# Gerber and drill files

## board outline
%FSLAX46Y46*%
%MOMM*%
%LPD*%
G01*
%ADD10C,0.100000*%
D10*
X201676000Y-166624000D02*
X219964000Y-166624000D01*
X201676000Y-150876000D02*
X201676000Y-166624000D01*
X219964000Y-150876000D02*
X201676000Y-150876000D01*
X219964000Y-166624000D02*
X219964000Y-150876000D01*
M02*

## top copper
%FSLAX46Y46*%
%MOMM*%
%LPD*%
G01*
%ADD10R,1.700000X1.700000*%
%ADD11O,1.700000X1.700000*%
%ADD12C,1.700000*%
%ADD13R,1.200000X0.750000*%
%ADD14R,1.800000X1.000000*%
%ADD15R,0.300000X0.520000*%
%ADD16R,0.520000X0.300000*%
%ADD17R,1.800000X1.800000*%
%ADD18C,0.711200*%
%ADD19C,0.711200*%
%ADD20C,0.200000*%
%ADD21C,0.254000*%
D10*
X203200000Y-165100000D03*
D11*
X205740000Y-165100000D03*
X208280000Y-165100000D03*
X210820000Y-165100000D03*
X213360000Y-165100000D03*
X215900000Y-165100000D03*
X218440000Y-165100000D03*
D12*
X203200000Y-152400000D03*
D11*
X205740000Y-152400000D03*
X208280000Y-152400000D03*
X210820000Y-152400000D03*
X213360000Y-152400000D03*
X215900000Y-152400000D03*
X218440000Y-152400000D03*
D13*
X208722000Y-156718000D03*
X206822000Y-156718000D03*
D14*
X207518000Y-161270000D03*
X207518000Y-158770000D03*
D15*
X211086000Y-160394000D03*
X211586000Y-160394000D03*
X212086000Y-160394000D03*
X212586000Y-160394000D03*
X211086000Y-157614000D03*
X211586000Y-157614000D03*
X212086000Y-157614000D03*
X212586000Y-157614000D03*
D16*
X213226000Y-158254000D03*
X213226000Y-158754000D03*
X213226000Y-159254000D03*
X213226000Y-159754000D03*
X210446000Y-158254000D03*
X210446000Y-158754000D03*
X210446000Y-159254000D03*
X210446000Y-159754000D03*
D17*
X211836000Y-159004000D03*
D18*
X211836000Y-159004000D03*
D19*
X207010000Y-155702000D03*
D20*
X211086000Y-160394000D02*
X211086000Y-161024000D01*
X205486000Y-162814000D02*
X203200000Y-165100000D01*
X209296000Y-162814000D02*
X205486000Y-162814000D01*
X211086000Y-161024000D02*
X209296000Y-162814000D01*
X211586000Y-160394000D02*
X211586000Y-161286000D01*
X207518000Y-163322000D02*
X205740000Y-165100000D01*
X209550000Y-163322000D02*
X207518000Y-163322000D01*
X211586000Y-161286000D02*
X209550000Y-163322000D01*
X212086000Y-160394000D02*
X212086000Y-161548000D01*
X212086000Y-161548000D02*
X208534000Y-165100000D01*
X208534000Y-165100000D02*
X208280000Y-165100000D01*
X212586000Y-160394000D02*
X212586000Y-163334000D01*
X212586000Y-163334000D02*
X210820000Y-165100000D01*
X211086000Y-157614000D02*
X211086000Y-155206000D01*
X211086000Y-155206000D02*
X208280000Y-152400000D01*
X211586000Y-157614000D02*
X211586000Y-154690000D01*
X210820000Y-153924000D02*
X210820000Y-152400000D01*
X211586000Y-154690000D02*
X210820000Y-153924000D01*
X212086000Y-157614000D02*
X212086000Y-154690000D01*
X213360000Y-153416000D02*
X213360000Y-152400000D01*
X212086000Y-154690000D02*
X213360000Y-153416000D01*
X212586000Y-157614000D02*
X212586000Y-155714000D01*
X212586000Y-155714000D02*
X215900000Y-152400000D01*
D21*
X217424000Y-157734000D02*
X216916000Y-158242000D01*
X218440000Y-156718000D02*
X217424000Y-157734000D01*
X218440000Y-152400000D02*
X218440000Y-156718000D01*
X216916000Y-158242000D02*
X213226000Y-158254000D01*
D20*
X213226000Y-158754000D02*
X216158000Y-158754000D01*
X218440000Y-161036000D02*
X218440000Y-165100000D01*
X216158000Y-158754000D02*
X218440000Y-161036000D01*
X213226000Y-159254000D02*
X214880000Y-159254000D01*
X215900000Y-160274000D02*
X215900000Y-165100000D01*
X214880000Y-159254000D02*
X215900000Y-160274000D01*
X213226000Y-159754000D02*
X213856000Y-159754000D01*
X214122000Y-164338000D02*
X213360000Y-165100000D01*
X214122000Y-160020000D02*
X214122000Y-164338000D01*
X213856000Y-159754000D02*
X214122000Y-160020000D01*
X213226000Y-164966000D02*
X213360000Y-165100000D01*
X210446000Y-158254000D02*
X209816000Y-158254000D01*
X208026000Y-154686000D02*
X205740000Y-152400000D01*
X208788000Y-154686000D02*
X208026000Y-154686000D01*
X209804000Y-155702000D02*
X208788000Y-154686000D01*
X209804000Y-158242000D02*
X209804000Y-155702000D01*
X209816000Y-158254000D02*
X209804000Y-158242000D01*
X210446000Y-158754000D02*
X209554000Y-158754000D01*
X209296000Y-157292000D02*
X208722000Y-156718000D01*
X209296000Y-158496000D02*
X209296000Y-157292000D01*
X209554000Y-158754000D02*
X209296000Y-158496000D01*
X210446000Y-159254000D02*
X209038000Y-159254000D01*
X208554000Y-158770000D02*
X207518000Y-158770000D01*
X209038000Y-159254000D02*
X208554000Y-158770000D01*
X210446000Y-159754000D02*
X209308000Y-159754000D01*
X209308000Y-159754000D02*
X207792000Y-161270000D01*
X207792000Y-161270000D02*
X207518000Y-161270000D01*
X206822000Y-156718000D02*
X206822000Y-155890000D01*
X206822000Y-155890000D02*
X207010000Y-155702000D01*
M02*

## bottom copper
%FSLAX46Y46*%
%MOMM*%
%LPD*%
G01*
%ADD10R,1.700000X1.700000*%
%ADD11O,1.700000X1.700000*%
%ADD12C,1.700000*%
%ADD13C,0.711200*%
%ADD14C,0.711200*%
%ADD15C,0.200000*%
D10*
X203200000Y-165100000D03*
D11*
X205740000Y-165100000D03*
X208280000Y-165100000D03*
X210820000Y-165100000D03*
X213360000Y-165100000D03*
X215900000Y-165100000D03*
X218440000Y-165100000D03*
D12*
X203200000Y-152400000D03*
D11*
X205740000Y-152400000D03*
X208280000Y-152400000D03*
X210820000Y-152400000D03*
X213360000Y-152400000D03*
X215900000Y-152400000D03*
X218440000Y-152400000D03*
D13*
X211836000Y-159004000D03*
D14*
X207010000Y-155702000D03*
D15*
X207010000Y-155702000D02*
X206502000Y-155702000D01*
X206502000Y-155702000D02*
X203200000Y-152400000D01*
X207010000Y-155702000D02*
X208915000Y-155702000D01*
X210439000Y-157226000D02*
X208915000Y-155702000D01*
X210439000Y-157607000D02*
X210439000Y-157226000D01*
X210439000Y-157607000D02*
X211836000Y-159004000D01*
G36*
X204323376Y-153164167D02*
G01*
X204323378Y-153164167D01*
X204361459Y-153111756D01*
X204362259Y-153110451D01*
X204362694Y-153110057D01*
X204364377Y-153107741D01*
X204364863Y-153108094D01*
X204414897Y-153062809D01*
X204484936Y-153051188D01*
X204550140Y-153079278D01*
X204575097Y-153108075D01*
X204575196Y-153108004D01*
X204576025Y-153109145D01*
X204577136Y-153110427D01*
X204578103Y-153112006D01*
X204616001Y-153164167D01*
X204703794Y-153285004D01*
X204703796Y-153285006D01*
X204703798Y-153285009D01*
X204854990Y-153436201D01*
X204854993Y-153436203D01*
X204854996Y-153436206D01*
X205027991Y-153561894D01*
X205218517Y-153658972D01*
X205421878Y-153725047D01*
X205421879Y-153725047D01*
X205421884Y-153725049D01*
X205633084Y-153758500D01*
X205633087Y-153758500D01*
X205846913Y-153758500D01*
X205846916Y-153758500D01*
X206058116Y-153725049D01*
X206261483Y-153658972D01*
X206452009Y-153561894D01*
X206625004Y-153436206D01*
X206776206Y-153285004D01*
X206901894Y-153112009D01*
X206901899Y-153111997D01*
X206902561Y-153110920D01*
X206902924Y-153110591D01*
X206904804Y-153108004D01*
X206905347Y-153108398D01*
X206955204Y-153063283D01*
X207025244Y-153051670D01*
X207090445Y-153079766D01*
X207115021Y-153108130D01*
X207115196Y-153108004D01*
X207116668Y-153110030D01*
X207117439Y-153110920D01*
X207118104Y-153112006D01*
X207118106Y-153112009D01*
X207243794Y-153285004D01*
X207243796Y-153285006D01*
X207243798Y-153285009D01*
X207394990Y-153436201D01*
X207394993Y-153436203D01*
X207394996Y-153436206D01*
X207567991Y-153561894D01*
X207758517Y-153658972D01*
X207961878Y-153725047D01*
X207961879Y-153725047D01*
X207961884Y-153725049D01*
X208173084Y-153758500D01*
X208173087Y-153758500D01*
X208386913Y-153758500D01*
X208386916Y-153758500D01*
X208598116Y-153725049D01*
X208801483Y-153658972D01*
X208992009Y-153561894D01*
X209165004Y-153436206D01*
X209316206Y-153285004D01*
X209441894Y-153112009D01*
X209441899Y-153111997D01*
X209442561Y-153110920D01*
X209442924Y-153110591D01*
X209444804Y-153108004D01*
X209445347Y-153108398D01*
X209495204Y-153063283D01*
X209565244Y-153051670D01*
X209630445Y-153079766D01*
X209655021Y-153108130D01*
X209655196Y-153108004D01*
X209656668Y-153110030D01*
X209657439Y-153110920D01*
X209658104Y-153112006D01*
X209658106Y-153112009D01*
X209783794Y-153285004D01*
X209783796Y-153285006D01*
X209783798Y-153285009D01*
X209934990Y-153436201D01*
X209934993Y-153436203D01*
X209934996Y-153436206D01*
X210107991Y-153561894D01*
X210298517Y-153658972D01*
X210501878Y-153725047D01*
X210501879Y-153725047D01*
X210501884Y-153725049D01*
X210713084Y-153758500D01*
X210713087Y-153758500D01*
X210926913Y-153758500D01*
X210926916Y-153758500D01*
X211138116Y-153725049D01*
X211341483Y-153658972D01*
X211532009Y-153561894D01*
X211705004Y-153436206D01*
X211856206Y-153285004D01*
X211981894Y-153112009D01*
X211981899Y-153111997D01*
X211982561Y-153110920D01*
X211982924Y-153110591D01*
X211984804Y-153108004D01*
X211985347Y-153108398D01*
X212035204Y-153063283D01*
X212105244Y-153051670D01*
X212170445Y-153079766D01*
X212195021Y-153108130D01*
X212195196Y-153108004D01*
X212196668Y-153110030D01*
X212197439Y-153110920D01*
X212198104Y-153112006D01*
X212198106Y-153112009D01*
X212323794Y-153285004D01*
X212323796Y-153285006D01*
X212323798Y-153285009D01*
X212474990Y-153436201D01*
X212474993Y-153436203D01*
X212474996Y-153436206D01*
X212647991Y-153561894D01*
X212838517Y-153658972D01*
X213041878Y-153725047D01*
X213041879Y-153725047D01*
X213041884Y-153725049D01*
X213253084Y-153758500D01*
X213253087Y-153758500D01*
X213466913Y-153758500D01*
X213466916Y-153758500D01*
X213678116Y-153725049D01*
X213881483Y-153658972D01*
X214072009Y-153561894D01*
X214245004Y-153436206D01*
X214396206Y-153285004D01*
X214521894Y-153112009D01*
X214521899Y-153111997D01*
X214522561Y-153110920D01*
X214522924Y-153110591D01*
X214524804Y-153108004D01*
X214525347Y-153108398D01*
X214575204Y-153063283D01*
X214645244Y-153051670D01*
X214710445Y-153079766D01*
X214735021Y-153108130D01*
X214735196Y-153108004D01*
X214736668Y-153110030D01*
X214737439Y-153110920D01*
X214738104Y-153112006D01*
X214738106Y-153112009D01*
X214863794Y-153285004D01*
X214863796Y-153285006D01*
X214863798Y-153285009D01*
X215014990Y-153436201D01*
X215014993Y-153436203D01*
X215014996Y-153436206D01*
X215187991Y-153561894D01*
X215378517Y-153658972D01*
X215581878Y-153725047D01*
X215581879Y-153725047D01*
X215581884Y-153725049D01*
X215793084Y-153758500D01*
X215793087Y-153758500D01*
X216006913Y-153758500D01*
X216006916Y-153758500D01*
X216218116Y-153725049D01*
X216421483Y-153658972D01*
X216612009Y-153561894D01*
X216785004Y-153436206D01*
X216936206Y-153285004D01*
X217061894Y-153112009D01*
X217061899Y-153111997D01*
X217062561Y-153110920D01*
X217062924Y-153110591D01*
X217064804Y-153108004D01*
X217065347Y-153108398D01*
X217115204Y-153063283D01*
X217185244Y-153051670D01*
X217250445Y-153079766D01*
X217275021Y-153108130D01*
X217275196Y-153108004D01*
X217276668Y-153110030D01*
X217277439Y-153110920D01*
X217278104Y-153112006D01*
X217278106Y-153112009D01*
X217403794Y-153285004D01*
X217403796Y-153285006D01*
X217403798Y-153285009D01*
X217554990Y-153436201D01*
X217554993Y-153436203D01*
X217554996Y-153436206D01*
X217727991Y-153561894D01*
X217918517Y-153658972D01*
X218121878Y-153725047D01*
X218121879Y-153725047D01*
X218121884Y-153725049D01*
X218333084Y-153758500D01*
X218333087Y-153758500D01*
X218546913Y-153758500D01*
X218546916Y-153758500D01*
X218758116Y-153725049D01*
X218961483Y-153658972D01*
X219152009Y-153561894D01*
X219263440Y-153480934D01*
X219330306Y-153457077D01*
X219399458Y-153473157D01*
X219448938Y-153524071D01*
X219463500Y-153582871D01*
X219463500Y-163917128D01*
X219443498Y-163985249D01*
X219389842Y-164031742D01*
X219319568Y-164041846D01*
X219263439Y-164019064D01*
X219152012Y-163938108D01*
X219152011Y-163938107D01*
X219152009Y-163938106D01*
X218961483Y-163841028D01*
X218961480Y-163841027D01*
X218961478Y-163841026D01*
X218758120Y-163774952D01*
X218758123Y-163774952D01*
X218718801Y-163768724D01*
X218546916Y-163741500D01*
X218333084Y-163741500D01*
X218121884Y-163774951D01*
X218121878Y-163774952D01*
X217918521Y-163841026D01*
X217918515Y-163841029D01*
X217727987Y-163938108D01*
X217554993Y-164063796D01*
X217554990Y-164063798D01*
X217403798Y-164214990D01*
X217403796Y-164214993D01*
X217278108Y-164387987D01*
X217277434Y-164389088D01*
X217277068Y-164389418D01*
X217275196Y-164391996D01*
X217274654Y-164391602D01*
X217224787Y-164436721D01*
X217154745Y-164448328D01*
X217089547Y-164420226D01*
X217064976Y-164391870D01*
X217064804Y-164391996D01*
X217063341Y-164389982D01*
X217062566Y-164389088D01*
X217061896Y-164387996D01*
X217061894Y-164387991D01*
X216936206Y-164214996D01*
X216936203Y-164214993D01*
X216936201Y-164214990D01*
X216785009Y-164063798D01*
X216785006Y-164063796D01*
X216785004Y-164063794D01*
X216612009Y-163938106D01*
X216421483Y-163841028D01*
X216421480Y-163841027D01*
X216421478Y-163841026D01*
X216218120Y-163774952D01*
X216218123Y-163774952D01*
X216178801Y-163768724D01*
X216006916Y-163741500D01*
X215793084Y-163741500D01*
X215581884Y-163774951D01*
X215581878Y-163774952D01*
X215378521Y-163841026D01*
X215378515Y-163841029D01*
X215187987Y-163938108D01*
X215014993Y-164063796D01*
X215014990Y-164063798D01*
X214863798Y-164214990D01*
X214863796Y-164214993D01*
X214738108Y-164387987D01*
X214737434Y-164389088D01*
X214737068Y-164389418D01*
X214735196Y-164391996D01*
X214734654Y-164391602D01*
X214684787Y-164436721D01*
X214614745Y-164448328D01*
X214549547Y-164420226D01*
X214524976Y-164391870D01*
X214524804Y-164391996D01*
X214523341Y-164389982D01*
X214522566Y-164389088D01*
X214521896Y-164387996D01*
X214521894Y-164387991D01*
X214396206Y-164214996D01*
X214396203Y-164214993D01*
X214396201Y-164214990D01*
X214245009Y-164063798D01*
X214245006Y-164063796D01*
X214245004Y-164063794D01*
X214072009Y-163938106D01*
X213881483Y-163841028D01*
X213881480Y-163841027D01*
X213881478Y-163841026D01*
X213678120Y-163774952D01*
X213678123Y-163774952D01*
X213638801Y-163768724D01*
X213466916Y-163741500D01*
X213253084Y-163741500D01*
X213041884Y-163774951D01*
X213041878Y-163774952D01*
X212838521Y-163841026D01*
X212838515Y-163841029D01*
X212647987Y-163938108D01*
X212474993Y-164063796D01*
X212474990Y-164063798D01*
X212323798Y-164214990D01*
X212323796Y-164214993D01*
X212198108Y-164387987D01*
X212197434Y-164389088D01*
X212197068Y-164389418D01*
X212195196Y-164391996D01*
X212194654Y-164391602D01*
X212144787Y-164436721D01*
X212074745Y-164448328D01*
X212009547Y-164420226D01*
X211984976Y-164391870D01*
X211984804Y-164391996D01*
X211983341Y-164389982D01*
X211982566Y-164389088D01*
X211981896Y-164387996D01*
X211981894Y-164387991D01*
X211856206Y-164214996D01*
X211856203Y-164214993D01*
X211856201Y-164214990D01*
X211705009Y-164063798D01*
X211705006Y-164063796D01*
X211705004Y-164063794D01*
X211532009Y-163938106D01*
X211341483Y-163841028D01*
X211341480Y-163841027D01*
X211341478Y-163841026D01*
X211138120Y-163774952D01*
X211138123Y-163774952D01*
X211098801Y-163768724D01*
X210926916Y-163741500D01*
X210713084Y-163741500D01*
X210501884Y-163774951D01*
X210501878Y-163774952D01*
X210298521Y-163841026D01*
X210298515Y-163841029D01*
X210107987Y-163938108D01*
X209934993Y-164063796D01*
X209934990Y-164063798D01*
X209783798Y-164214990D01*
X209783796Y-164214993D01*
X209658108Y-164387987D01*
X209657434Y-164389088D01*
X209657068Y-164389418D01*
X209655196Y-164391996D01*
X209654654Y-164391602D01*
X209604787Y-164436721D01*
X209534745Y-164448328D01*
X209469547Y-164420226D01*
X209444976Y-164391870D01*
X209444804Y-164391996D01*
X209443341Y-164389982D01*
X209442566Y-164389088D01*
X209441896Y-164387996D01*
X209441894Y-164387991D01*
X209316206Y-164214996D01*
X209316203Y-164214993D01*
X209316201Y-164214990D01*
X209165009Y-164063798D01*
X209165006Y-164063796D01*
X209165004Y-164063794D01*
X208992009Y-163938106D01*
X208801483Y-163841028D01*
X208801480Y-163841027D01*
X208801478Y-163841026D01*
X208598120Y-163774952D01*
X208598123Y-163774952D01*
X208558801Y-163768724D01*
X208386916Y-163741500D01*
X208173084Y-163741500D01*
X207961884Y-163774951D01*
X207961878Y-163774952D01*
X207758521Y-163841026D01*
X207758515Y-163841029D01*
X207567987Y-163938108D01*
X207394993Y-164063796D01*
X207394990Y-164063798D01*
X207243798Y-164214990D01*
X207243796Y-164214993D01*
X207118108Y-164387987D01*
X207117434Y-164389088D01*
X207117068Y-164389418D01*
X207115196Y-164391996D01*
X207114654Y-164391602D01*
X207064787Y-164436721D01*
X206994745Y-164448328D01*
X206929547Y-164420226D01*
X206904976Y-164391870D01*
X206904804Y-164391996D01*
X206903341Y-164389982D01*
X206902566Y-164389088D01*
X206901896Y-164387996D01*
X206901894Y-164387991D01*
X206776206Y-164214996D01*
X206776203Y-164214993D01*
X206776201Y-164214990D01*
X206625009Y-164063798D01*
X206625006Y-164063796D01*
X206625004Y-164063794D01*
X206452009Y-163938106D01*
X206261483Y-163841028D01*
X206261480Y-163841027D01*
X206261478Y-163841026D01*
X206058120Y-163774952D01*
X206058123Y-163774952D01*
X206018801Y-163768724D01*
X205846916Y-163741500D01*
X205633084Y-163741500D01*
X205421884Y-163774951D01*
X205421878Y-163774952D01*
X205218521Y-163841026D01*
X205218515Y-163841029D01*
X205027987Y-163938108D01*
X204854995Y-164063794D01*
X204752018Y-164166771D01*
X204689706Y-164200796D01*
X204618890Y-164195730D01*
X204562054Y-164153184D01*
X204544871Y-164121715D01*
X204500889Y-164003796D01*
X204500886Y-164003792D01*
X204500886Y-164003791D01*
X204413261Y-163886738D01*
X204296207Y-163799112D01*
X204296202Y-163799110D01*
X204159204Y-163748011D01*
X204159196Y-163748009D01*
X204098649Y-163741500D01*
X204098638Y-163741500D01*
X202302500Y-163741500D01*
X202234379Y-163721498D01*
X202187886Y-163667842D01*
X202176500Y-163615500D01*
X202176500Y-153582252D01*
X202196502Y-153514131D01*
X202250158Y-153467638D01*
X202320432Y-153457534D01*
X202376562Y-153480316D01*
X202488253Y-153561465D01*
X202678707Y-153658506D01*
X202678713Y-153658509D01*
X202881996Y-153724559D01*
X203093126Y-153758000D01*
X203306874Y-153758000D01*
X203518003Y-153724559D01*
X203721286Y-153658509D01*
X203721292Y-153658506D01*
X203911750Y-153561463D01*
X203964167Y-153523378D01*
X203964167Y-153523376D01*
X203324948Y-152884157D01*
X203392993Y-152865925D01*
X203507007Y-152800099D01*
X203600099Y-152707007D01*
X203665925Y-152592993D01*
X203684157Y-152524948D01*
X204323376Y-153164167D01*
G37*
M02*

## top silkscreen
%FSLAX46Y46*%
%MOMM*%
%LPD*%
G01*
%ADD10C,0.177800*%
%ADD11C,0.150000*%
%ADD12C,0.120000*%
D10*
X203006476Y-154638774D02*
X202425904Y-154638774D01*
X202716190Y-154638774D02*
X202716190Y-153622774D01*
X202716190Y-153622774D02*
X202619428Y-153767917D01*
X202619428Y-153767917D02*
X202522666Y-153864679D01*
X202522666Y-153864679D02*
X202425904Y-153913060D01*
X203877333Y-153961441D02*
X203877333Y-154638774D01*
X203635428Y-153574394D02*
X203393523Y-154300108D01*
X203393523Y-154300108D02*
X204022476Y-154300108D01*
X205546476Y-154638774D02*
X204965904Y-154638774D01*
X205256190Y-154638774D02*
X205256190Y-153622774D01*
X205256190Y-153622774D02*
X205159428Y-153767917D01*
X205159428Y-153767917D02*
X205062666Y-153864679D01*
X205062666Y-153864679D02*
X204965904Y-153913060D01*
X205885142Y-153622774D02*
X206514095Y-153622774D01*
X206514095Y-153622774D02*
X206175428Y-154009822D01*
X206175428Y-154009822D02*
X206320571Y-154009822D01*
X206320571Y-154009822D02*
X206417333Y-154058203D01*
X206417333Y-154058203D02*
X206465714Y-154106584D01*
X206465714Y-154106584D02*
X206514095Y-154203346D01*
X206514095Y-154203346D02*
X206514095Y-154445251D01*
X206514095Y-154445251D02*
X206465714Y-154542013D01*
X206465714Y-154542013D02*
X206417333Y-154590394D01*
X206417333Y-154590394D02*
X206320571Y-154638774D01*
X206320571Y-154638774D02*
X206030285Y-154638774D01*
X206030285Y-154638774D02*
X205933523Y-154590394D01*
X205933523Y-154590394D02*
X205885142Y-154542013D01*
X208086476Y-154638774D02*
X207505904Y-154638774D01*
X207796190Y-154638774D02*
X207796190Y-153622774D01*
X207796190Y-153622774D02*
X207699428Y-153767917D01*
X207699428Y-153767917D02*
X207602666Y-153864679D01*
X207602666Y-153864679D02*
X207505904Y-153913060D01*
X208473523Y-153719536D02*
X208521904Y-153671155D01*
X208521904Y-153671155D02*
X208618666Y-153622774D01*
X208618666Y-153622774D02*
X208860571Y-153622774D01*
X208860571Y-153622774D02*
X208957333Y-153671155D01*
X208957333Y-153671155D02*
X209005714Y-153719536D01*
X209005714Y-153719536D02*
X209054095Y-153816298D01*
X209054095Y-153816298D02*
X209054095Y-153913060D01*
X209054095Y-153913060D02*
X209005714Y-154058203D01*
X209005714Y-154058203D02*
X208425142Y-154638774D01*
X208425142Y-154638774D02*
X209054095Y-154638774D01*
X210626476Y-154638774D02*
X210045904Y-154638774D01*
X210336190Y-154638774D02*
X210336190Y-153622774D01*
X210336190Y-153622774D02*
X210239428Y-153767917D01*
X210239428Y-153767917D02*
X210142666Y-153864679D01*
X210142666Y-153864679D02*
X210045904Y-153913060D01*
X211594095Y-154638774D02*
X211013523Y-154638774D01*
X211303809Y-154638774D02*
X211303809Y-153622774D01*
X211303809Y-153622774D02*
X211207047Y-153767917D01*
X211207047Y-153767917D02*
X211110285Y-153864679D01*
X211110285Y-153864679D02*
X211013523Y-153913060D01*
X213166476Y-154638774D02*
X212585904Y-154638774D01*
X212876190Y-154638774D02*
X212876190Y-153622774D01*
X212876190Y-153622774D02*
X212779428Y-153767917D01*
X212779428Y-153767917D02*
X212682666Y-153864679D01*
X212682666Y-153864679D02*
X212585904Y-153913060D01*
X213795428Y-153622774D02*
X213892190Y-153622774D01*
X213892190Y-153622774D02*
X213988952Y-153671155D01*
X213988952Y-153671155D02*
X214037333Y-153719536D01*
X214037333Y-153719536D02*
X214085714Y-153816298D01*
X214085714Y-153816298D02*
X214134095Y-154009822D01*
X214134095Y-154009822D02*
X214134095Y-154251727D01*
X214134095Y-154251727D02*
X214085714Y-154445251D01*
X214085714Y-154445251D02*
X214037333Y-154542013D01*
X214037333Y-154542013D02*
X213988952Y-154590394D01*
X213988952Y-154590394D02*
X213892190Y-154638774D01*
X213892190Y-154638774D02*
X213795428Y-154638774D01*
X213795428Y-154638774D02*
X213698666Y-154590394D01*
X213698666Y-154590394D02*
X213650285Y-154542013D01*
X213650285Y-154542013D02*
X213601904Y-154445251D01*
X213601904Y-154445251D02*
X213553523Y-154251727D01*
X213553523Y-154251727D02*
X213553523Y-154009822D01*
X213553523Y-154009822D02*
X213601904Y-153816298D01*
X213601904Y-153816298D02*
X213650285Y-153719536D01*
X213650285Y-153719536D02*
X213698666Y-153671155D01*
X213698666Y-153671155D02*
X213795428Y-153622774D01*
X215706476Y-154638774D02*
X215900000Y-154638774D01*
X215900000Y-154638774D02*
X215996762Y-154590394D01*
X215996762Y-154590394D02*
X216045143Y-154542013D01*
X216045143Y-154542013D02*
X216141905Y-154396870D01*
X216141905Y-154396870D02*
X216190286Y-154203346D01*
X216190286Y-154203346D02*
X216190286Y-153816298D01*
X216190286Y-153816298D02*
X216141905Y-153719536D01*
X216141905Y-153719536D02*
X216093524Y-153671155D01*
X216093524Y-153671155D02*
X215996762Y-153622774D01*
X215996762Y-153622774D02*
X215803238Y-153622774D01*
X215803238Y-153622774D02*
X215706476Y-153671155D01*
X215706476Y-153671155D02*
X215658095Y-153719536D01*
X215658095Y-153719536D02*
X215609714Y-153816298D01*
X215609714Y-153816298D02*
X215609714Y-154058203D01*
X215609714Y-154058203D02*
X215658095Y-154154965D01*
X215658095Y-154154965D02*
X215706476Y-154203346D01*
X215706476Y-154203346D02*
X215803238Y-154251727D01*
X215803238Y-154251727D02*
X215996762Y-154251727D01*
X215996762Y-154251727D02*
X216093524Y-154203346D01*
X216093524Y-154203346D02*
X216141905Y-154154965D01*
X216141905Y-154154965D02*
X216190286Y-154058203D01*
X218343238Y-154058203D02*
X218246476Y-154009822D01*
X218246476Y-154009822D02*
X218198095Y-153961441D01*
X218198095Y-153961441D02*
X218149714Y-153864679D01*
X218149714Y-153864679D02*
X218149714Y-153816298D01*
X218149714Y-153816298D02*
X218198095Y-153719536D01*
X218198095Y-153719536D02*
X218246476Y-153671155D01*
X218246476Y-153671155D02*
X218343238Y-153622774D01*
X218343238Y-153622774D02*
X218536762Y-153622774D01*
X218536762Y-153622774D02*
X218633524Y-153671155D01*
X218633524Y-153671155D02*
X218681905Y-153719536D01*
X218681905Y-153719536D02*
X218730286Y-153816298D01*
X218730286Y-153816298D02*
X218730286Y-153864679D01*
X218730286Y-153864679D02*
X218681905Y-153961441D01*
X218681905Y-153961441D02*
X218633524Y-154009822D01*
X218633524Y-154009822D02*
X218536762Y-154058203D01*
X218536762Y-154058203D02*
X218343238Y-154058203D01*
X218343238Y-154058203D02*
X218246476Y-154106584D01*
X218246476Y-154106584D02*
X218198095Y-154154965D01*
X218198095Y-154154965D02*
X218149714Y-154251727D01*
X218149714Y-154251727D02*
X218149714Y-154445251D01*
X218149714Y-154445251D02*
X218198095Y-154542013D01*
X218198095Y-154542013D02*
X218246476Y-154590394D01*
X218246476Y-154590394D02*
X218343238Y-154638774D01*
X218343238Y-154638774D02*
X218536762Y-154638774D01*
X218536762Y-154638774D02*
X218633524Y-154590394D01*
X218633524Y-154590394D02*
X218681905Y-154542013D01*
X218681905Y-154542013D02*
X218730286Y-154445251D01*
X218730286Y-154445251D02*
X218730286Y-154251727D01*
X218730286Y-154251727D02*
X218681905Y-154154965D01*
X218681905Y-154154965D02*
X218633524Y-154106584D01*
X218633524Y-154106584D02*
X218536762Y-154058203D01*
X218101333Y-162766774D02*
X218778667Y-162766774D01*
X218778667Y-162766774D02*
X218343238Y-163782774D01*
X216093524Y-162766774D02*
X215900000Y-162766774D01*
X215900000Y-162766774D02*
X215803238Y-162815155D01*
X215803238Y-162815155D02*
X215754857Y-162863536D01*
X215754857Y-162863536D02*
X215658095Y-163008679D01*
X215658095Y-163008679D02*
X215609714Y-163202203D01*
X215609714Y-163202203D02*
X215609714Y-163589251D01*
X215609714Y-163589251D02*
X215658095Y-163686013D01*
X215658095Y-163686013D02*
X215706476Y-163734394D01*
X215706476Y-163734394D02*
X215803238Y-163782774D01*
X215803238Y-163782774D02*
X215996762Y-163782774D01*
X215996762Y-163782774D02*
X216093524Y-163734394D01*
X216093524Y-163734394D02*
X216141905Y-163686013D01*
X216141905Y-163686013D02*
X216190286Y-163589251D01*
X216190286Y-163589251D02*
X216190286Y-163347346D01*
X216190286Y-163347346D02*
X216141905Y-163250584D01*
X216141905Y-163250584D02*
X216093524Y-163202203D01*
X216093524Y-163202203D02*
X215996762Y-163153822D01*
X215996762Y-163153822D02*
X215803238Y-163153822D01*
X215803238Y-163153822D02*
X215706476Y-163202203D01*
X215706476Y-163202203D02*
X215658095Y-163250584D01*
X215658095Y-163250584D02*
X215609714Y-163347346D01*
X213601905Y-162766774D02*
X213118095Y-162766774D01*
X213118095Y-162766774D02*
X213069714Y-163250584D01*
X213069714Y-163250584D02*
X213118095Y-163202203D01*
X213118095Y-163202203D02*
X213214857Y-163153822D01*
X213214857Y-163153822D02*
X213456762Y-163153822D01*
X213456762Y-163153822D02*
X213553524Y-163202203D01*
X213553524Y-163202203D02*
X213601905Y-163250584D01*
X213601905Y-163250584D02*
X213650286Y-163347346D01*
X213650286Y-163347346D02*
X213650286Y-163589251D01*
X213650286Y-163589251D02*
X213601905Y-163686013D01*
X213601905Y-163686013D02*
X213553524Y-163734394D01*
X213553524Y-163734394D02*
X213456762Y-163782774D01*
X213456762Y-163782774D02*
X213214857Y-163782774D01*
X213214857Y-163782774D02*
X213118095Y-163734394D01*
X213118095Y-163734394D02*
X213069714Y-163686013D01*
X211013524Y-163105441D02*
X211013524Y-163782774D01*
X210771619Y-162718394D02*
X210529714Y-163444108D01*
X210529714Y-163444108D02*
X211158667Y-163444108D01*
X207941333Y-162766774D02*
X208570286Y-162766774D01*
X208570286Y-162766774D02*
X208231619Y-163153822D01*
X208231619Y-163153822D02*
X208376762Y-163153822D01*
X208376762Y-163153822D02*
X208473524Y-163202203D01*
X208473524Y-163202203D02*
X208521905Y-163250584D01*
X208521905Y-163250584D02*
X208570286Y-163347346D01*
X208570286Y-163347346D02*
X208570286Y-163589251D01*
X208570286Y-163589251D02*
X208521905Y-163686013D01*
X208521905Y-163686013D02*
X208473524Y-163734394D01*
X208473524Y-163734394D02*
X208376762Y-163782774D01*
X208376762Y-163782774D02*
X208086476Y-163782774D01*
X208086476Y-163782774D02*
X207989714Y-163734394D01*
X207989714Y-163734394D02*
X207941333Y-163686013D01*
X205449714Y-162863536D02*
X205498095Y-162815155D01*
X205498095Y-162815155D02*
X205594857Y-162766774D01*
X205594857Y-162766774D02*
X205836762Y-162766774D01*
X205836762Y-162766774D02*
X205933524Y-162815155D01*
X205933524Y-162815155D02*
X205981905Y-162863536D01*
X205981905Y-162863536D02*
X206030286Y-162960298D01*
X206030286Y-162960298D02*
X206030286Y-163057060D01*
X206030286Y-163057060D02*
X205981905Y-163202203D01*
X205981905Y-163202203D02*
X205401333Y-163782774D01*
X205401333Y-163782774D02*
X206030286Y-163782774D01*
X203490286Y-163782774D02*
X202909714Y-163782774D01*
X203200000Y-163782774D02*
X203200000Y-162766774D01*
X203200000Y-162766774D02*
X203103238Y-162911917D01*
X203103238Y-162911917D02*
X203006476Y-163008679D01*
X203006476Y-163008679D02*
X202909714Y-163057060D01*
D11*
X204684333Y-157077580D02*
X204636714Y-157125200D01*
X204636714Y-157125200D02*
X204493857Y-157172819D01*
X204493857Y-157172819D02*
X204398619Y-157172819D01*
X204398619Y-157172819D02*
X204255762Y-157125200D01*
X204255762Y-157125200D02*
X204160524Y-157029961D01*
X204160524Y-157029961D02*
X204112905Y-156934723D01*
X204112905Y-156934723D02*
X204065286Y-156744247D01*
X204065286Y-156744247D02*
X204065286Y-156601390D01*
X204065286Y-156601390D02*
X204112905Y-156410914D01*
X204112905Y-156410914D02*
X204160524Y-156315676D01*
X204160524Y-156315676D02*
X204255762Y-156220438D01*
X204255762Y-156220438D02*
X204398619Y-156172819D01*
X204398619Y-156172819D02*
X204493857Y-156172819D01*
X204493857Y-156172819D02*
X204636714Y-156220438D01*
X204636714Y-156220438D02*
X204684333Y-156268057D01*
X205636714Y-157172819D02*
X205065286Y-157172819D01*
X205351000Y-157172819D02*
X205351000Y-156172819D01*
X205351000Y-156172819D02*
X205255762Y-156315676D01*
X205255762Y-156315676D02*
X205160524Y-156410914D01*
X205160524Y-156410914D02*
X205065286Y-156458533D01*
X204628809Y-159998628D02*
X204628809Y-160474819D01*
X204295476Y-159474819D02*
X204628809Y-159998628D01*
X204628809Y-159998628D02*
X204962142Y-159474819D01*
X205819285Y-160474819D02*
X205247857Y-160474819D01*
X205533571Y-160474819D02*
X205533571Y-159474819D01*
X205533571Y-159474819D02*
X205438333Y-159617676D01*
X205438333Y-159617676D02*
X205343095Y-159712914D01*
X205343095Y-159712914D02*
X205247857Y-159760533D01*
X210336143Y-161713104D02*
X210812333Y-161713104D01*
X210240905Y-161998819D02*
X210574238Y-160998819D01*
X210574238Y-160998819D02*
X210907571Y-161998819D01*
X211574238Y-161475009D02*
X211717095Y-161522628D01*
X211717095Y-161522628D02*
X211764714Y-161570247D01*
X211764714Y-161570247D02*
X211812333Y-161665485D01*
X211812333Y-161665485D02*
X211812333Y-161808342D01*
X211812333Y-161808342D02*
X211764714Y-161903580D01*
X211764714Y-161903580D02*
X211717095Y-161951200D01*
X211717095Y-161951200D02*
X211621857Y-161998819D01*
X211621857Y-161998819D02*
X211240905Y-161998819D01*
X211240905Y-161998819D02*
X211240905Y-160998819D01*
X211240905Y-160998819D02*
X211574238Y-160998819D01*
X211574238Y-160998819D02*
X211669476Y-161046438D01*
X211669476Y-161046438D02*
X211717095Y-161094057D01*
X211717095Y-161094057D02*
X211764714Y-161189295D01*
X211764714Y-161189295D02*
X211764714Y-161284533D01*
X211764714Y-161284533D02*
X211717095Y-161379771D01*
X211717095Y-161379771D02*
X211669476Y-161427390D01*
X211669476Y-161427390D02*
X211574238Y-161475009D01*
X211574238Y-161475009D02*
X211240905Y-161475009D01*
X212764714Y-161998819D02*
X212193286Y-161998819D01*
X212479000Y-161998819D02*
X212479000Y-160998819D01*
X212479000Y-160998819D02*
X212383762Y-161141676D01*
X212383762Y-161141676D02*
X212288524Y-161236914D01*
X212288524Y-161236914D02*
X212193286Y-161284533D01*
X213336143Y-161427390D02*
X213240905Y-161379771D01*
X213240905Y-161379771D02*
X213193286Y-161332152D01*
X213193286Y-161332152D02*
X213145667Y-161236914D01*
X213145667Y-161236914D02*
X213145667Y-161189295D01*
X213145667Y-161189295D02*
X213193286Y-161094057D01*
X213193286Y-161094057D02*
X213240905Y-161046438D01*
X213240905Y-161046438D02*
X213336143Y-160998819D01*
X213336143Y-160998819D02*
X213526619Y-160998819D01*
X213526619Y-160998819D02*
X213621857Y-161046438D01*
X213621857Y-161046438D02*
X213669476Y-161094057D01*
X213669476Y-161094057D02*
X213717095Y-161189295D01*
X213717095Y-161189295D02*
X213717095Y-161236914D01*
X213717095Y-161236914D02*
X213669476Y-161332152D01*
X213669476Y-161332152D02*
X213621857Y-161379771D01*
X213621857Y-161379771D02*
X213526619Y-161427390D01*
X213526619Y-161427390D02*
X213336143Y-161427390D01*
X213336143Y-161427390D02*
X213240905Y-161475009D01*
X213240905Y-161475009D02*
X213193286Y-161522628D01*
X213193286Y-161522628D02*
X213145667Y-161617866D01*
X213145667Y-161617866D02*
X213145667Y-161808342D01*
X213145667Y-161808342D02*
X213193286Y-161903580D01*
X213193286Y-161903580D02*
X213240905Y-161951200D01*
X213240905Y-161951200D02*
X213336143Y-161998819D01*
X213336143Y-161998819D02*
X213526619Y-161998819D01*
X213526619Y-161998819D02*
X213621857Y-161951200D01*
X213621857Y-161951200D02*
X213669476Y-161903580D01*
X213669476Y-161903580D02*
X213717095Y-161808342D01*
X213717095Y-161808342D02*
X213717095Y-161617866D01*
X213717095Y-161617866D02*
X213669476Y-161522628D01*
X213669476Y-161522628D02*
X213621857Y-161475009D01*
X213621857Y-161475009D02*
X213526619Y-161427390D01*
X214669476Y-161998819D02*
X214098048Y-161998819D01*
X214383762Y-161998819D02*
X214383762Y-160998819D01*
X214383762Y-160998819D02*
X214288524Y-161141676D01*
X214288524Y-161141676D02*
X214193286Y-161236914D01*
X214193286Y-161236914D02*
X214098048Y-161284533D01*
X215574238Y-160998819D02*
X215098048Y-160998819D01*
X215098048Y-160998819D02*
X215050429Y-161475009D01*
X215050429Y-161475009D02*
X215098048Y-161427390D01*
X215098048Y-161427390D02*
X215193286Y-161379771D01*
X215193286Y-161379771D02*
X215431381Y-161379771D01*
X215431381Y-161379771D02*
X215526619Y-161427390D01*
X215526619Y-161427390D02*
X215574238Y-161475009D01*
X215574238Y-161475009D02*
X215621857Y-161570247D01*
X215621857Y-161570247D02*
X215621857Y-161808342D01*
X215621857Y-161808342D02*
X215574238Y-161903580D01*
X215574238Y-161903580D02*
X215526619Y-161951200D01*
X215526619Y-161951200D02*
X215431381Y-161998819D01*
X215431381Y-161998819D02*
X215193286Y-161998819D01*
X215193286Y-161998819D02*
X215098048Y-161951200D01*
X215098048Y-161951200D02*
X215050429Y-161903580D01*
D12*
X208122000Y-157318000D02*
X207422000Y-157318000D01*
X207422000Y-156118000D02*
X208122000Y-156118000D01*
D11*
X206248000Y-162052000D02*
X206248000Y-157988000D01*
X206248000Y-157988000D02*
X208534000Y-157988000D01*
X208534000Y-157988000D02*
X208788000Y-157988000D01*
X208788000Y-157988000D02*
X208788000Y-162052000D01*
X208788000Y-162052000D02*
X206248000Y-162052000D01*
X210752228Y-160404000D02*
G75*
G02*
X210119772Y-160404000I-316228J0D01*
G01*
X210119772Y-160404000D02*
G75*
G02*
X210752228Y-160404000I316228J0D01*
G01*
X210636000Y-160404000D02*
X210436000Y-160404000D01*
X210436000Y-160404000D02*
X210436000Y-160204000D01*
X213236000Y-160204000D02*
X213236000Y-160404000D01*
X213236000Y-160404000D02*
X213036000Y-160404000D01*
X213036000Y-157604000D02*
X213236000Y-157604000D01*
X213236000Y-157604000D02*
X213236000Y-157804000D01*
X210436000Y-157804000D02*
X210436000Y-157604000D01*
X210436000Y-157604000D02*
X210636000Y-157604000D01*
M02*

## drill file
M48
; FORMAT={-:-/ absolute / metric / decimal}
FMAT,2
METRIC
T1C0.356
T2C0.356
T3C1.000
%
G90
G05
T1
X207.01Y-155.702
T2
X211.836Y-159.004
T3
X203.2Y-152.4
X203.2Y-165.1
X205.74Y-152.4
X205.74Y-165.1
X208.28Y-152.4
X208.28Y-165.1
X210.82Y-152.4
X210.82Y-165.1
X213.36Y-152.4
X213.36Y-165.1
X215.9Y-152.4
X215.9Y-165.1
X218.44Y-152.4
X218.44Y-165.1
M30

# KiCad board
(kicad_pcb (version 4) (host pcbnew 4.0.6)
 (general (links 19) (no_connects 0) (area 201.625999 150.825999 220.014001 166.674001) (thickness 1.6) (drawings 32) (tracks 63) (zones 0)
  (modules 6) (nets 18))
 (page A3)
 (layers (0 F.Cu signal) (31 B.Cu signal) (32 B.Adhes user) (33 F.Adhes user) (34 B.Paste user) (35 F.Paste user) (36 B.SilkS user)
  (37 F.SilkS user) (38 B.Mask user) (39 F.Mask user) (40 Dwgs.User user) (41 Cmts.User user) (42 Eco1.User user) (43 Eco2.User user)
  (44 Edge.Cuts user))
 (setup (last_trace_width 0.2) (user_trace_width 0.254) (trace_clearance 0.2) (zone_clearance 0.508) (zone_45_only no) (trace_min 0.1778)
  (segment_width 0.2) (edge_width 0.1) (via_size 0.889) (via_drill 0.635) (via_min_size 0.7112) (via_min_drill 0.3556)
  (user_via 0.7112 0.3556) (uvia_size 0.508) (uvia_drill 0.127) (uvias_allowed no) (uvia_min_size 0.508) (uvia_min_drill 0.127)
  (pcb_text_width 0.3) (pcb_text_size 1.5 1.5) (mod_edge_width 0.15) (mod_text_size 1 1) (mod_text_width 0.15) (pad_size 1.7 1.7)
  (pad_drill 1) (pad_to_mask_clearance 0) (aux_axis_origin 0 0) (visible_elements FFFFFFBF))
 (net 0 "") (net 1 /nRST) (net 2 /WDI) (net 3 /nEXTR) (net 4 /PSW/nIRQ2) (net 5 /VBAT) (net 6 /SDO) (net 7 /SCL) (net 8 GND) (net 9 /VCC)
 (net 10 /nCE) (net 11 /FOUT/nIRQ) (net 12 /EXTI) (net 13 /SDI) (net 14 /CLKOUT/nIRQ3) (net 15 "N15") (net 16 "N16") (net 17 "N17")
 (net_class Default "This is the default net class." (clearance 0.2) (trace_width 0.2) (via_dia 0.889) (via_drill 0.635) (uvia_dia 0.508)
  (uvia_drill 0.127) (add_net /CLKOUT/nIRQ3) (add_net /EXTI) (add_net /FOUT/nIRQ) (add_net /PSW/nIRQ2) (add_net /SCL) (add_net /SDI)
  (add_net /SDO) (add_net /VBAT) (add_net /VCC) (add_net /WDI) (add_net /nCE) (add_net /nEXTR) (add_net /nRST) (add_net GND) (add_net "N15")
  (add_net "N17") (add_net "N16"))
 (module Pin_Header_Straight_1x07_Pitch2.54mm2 (layer F.Cu) (at 203.2 165.1 90)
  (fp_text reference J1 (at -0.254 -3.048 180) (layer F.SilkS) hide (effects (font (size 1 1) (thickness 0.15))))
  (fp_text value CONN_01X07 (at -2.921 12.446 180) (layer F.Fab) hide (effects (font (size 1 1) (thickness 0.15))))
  (pad 1 thru_hole rect (at 0 0 90) (size 1.7 1.7) (drill 1) (layers *.Cu *.Mask) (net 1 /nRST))
  (pad 2 thru_hole oval (at 0 2.54 90) (size 1.7 1.7) (drill 1) (layers *.Cu *.Mask) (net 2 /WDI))
  (pad 3 thru_hole oval (at 0 5.08 90) (size 1.7 1.7) (drill 1) (layers *.Cu *.Mask) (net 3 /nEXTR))
  (pad 4 thru_hole oval (at 0 7.62 90) (size 1.7 1.7) (drill 1) (layers *.Cu *.Mask) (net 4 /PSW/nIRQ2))
  (pad 5 thru_hole oval (at 0 10.16 90) (size 1.7 1.7) (drill 1) (layers *.Cu *.Mask) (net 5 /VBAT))
  (pad 6 thru_hole oval (at 0 12.7 90) (size 1.7 1.7) (drill 1) (layers *.Cu *.Mask) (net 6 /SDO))
  (pad 7 thru_hole oval (at 0 15.24 90) (size 1.7 1.7) (drill 1) (layers *.Cu *.Mask) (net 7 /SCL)))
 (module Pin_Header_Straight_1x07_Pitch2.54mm (layer F.Cu) (at 203.2 152.4 90)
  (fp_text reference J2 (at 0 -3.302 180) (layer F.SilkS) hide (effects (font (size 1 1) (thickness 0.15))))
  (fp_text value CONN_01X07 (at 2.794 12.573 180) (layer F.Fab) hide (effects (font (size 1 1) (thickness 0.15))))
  (pad 1 thru_hole circle (at 0 0 90) (size 1.7 1.7) (drill 1) (layers *.Cu *.Mask) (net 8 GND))
  (pad 2 thru_hole oval (at 0 2.54 90) (size 1.7 1.7) (drill 1) (layers *.Cu *.Mask) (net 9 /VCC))
  (pad 3 thru_hole oval (at 0 5.08 90) (size 1.7 1.7) (drill 1) (layers *.Cu *.Mask) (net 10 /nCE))
  (pad 4 thru_hole oval (at 0 7.62 90) (size 1.7 1.7) (drill 1) (layers *.Cu *.Mask) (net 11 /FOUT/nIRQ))
  (pad 5 thru_hole oval (at 0 10.16 90) (size 1.7 1.7) (drill 1) (layers *.Cu *.Mask) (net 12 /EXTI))
  (pad 6 thru_hole oval (at 0 12.7 90) (size 1.7 1.7) (drill 1) (layers *.Cu *.Mask) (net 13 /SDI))
  (pad 7 thru_hole oval (at 0 15.24 90) (size 1.7 1.7) (drill 1) (layers *.Cu *.Mask) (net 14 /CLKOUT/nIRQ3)))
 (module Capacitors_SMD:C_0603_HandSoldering (layer F.Cu) (at 207.772 156.718 180)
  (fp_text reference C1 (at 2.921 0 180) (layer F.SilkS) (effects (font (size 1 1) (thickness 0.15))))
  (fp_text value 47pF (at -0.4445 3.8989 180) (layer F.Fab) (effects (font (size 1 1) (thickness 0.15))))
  (fp_line (start -0.35 -0.6) (end 0.35 -0.6) (layer F.SilkS) (width 0.12))
  (fp_line (start 0.35 0.6) (end -0.35 0.6) (layer F.SilkS) (width 0.12))
  (pad 1 smd rect (at -0.95 0 180) (size 1.2 0.75) (layers F.Cu F.Paste F.Mask) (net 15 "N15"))
  (pad 2 smd rect (at 0.95 0 180) (size 1.2 0.75) (layers F.Cu F.Paste F.Mask) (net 8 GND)))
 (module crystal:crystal (layer F.Cu) (at 207.518 160.02 90)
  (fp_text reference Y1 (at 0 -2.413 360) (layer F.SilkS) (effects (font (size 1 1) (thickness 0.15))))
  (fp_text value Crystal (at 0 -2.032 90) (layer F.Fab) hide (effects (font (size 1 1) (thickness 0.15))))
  (fp_line (start -2.032 -1.27) (end 2.032 -1.27) (layer F.SilkS) (width 0.15))
  (fp_line (start 2.032 -1.27) (end 2.032 1.016) (layer F.SilkS) (width 0.15))
  (fp_line (start 2.032 1.016) (end 2.032 1.27) (layer F.SilkS) (width 0.15))
  (fp_line (start 2.032 1.27) (end -2.032 1.27) (layer F.SilkS) (width 0.15))
  (fp_line (start -2.032 1.27) (end -2.032 -1.27) (layer F.SilkS) (width 0.15))
  (pad 1 smd rect (at -1.25 0 90) (size 1 1.8) (layers F.Cu F.Paste F.Mask) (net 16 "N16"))
  (pad 2 smd rect (at 1.25 0 90) (size 1 1.8) (layers F.Cu F.Paste F.Mask) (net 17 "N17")))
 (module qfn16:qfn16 (layer F.Cu) (at 211.836 159.004) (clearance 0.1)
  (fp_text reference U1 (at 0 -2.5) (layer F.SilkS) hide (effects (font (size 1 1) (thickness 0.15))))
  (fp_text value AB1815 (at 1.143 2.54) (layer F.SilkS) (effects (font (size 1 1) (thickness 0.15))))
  (fp_circle (center -1.4 1.4) (end -1.1 1.5) (layer F.SilkS) (width 0.15))
  (fp_line (start -1.2 1.4) (end -1.4 1.4) (layer F.SilkS) (width 0.15))
  (fp_line (start -1.4 1.4) (end -1.4 1.2) (layer F.SilkS) (width 0.15))
  (fp_line (start 1.4 1.2) (end 1.4 1.4) (layer F.SilkS) (width 0.15))
  (fp_line (start 1.4 1.4) (end 1.2 1.4) (layer F.SilkS) (width 0.15))
  (fp_line (start 1.2 -1.4) (end 1.4 -1.4) (layer F.SilkS) (width 0.15))
  (fp_line (start 1.4 -1.4) (end 1.4 -1.2) (layer F.SilkS) (width 0.15))
  (fp_line (start -1.4 -1.2) (end -1.4 -1.4) (layer F.SilkS) (width 0.15))
  (fp_line (start -1.4 -1.4) (end -1.2 -1.4) (layer F.SilkS) (width 0.15))
  (pad 1 smd rect (at -0.75 1.39 180) (size 0.3 0.52) (layers F.Cu F.Paste F.Mask) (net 1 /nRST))
  (pad 2 smd rect (at -0.25 1.39 180) (size 0.3 0.52) (layers F.Cu F.Paste F.Mask) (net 2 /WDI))
  (pad 3 smd rect (at 0.25 1.39 180) (size 0.3 0.52) (layers F.Cu F.Paste F.Mask) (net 3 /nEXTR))
  (pad 4 smd rect (at 0.75 1.39 180) (size 0.3 0.52) (layers F.Cu F.Paste F.Mask) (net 4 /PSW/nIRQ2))
  (pad 12 smd rect (at -0.75 -1.39 180) (size 0.3 0.52) (layers F.Cu F.Paste F.Mask) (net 10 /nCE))
  (pad 11 smd rect (at -0.25 -1.39 180) (size 0.3 0.52) (layers F.Cu F.Paste F.Mask) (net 11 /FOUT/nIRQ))
  (pad 10 smd rect (at 0.25 -1.39 180) (size 0.3 0.52) (layers F.Cu F.Paste F.Mask) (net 12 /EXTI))
  (pad 9 smd rect (at 0.75 -1.39 180) (size 0.3 0.52) (layers F.Cu F.Paste F.Mask) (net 13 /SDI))
  (pad 8 smd rect (at 1.39 -0.75 180) (size 0.52 0.3) (layers F.Cu F.Paste F.Mask) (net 14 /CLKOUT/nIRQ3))
  (pad 7 smd rect (at 1.39 -0.25 180) (size 0.52 0.3) (layers F.Cu F.Paste F.Mask) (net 7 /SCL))
  (pad 6 smd rect (at 1.39 0.25 180) (size 0.52 0.3) (layers F.Cu F.Paste F.Mask) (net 6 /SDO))
  (pad 5 smd rect (at 1.39 0.75 180) (size 0.52 0.3) (layers F.Cu F.Paste F.Mask) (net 5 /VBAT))
  (pad 13 smd rect (at -1.39 -0.75 180) (size 0.52 0.3) (layers F.Cu F.Paste F.Mask) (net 9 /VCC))
  (pad 14 smd rect (at -1.39 -0.25 180) (size 0.52 0.3) (layers F.Cu F.Paste F.Mask) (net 15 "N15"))
  (pad 15 smd rect (at -1.39 0.25 180) (size 0.52 0.3) (layers F.Cu F.Paste F.Mask) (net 17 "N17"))
  (pad 16 smd rect (at -1.39 0.75 180) (size 0.52 0.3) (layers F.Cu F.Paste F.Mask) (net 16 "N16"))
  (pad PAD smd rect (at 0 0 180) (size 1.8 1.8) (layers F.Cu F.Paste F.Mask) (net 8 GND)))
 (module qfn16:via (layer F.Cu) (at 211.836 159.004)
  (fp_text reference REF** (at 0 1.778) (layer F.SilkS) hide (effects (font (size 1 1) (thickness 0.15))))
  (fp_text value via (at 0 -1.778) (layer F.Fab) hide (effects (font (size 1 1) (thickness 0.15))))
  (pad 1 thru_hole circle (at 0 0) (size 0.7112 0.7112) (drill 0.3556) (layers *.Cu) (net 8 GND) (zone_connect 2)))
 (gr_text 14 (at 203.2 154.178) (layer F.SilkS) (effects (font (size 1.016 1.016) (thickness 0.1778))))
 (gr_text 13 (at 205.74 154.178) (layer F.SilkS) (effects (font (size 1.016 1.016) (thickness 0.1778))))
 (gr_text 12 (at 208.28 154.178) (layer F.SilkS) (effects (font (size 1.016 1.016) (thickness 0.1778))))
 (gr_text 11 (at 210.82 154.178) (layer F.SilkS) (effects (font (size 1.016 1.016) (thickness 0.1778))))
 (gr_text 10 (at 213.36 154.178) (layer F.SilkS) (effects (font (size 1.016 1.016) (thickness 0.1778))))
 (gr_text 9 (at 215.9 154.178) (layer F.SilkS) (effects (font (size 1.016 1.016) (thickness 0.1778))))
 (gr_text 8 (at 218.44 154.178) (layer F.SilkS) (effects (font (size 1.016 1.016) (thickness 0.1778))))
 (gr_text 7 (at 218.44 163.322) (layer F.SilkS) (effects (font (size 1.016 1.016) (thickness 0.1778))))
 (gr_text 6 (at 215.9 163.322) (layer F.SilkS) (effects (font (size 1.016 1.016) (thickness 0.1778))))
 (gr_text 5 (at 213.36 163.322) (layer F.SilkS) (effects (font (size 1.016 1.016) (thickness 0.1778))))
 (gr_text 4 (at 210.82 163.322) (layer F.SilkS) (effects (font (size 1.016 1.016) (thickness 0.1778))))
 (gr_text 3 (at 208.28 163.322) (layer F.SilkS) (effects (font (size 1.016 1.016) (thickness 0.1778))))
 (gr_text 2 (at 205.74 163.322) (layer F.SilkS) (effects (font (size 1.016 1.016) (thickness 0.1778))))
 (gr_line (start 201.676 166.624) (end 219.964 166.624) (angle 90) (layer Edge.Cuts) (width 0.1))
 (gr_line (start 201.676 150.876) (end 201.676 166.624) (angle 90) (layer Edge.Cuts) (width 0.1))
 (gr_line (start 219.964 150.876) (end 201.676 150.876) (angle 90) (layer Edge.Cuts) (width 0.1))
 (gr_line (start 219.964 166.624) (end 219.964 150.876) (angle 90) (layer Edge.Cuts) (width 0.1))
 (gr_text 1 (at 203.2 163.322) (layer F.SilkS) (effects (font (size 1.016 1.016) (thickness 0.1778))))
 (segment (start 211.086 160.394) (end 211.086 161.024) (width 0.2) (layer F.Cu) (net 1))
 (segment (start 205.486 162.814) (end 203.2 165.1) (width 0.2) (layer F.Cu) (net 1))
 (segment (start 209.296 162.814) (end 205.486 162.814) (width 0.2) (layer F.Cu) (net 1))
 (segment (start 211.086 161.024) (end 209.296 162.814) (width 0.2) (layer F.Cu) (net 1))
 (segment (start 211.586 160.394) (end 211.586 161.286) (width 0.2) (layer F.Cu) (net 2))
 (segment (start 207.518 163.322) (end 205.74 165.1) (width 0.2) (layer F.Cu) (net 2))
 (segment (start 209.55 163.322) (end 207.518 163.322) (width 0.2) (layer F.Cu) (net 2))
 (segment (start 211.586 161.286) (end 209.55 163.322) (width 0.2) (layer F.Cu) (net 2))
 (segment (start 212.086 160.394) (end 212.086 161.548) (width 0.2) (layer F.Cu) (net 3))
 (segment (start 212.086 161.548) (end 208.534 165.1) (width 0.2) (layer F.Cu) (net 3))
 (segment (start 208.534 165.1) (end 208.28 165.1) (width 0.2) (layer F.Cu) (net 3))
 (segment (start 212.586 160.394) (end 212.586 163.334) (width 0.2) (layer F.Cu) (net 4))
 (segment (start 212.586 163.334) (end 210.82 165.1) (width 0.2) (layer F.Cu) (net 4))
 (segment (start 211.086 157.614) (end 211.086 155.206) (width 0.2) (layer F.Cu) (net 10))
 (segment (start 211.086 155.206) (end 208.28 152.4) (width 0.2) (layer F.Cu) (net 10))
 (segment (start 211.586 157.614) (end 211.586 154.69) (width 0.2) (layer F.Cu) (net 11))
 (segment (start 210.82 153.924) (end 210.82 152.4) (width 0.2) (layer F.Cu) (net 11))
 (segment (start 211.586 154.69) (end 210.82 153.924) (width 0.2) (layer F.Cu) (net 11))
 (segment (start 212.086 157.614) (end 212.086 154.69) (width 0.2) (layer F.Cu) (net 12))
 (segment (start 213.36 153.416) (end 213.36 152.4) (width 0.2) (layer F.Cu) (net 12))
 (segment (start 212.086 154.69) (end 213.36 153.416) (width 0.2) (layer F.Cu) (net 12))
 (segment (start 212.586 157.614) (end 212.586 155.714) (width 0.2) (layer F.Cu) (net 13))
 (segment (start 212.586 155.714) (end 215.9 152.4) (width 0.2) (layer F.Cu) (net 13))
 (segment (start 217.424 157.734) (end 216.916 158.242) (width 0.254) (layer F.Cu) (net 14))
 (segment (start 218.44 156.718) (end 217.424 157.734) (width 0.254) (layer F.Cu) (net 14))
 (segment (start 218.44 152.4) (end 218.44 156.718) (width 0.254) (layer F.Cu) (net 14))
 (segment (start 216.916 158.242) (end 213.226 158.254) (width 0.254) (layer F.Cu) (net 14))
 (segment (start 213.226 158.754) (end 216.158 158.754) (width 0.2) (layer F.Cu) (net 7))
 (segment (start 218.44 161.036) (end 218.44 165.1) (width 0.2) (layer F.Cu) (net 7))
 (segment (start 216.158 158.754) (end 218.44 161.036) (width 0.2) (layer F.Cu) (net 7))
 (segment (start 213.226 159.254) (end 214.88 159.254) (width 0.2) (layer F.Cu) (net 6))
 (segment (start 215.9 160.274) (end 215.9 165.1) (width 0.2) (layer F.Cu) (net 6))
 (segment (start 214.88 159.254) (end 215.9 160.274) (width 0.2) (layer F.Cu) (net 6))
 (segment (start 213.226 159.754) (end 213.856 159.754) (width 0.2) (layer F.Cu) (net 5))
 (segment (start 214.122 164.338) (end 213.36 165.1) (width 0.2) (layer F.Cu) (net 5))
 (segment (start 214.122 160.02) (end 214.122 164.338) (width 0.2) (layer F.Cu) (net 5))
 (segment (start 213.856 159.754) (end 214.122 160.02) (width 0.2) (layer F.Cu) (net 5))
 (segment (start 213.226 164.966) (end 213.36 165.1) (width 0.2) (layer F.Cu) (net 5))
 (segment (start 210.446 158.254) (end 209.816 158.254) (width 0.2) (layer F.Cu) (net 9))
 (segment (start 208.026 154.686) (end 205.74 152.4) (width 0.2) (layer F.Cu) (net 9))
 (segment (start 208.788 154.686) (end 208.026 154.686) (width 0.2) (layer F.Cu) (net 9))
 (segment (start 209.804 155.702) (end 208.788 154.686) (width 0.2) (layer F.Cu) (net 9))
 (segment (start 209.804 158.242) (end 209.804 155.702) (width 0.2) (layer F.Cu) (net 9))
 (segment (start 209.816 158.254) (end 209.804 158.242) (width 0.2) (layer F.Cu) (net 9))
 (segment (start 210.446 158.754) (end 209.554 158.754) (width 0.2) (layer F.Cu) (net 15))
 (segment (start 209.296 157.292) (end 208.722 156.718) (width 0.2) (layer F.Cu) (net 15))
 (segment (start 209.296 158.496) (end 209.296 157.292) (width 0.2) (layer F.Cu) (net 15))
 (segment (start 209.554 158.754) (end 209.296 158.496) (width 0.2) (layer F.Cu) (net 15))
 (segment (start 210.446 159.254) (end 209.038 159.254) (width 0.2) (layer F.Cu) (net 17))
 (segment (start 208.554 158.77) (end 207.518 158.77) (width 0.2) (layer F.Cu) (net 17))
 (segment (start 209.038 159.254) (end 208.554 158.77) (width 0.2) (layer F.Cu) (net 17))
 (segment (start 210.446 159.754) (end 209.308 159.754) (width 0.2) (layer F.Cu) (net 16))
 (segment (start 209.308 159.754) (end 207.792 161.27) (width 0.2) (layer F.Cu) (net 16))
 (segment (start 207.792 161.27) (end 207.518 161.27) (width 0.2) (layer F.Cu) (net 16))
 (segment (start 207.01 155.702) (end 206.502 155.702) (width 0.2) (layer B.Cu) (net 8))
 (segment (start 206.502 155.702) (end 203.2 152.4) (width 0.2) (layer B.Cu) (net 8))
 (segment (start 207.01 155.702) (end 208.915 155.702) (width 0.2) (layer B.Cu) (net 8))
 (segment (start 210.439 157.226) (end 208.915 155.702) (width 0.2) (layer B.Cu) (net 8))
 (segment (start 210.439 157.607) (end 210.439 157.226) (width 0.2) (layer B.Cu) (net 8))
 (segment (start 210.439 157.607) (end 211.836 159.004) (width 0.2) (layer B.Cu) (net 8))
 (via (at 207.01 155.702) (size 0.7112) (drill 0.3556) (layers F.Cu B.Cu) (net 8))
 (segment (start 206.822 156.718) (end 206.822 155.89) (width 0.2) (layer F.Cu) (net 8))
 (segment (start 206.822 155.89) (end 207.01 155.702) (width 0.2) (layer F.Cu) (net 8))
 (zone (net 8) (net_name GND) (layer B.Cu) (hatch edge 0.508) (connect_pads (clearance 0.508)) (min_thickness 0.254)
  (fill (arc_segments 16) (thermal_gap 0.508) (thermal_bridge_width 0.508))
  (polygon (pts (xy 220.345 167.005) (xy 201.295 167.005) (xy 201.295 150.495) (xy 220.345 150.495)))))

